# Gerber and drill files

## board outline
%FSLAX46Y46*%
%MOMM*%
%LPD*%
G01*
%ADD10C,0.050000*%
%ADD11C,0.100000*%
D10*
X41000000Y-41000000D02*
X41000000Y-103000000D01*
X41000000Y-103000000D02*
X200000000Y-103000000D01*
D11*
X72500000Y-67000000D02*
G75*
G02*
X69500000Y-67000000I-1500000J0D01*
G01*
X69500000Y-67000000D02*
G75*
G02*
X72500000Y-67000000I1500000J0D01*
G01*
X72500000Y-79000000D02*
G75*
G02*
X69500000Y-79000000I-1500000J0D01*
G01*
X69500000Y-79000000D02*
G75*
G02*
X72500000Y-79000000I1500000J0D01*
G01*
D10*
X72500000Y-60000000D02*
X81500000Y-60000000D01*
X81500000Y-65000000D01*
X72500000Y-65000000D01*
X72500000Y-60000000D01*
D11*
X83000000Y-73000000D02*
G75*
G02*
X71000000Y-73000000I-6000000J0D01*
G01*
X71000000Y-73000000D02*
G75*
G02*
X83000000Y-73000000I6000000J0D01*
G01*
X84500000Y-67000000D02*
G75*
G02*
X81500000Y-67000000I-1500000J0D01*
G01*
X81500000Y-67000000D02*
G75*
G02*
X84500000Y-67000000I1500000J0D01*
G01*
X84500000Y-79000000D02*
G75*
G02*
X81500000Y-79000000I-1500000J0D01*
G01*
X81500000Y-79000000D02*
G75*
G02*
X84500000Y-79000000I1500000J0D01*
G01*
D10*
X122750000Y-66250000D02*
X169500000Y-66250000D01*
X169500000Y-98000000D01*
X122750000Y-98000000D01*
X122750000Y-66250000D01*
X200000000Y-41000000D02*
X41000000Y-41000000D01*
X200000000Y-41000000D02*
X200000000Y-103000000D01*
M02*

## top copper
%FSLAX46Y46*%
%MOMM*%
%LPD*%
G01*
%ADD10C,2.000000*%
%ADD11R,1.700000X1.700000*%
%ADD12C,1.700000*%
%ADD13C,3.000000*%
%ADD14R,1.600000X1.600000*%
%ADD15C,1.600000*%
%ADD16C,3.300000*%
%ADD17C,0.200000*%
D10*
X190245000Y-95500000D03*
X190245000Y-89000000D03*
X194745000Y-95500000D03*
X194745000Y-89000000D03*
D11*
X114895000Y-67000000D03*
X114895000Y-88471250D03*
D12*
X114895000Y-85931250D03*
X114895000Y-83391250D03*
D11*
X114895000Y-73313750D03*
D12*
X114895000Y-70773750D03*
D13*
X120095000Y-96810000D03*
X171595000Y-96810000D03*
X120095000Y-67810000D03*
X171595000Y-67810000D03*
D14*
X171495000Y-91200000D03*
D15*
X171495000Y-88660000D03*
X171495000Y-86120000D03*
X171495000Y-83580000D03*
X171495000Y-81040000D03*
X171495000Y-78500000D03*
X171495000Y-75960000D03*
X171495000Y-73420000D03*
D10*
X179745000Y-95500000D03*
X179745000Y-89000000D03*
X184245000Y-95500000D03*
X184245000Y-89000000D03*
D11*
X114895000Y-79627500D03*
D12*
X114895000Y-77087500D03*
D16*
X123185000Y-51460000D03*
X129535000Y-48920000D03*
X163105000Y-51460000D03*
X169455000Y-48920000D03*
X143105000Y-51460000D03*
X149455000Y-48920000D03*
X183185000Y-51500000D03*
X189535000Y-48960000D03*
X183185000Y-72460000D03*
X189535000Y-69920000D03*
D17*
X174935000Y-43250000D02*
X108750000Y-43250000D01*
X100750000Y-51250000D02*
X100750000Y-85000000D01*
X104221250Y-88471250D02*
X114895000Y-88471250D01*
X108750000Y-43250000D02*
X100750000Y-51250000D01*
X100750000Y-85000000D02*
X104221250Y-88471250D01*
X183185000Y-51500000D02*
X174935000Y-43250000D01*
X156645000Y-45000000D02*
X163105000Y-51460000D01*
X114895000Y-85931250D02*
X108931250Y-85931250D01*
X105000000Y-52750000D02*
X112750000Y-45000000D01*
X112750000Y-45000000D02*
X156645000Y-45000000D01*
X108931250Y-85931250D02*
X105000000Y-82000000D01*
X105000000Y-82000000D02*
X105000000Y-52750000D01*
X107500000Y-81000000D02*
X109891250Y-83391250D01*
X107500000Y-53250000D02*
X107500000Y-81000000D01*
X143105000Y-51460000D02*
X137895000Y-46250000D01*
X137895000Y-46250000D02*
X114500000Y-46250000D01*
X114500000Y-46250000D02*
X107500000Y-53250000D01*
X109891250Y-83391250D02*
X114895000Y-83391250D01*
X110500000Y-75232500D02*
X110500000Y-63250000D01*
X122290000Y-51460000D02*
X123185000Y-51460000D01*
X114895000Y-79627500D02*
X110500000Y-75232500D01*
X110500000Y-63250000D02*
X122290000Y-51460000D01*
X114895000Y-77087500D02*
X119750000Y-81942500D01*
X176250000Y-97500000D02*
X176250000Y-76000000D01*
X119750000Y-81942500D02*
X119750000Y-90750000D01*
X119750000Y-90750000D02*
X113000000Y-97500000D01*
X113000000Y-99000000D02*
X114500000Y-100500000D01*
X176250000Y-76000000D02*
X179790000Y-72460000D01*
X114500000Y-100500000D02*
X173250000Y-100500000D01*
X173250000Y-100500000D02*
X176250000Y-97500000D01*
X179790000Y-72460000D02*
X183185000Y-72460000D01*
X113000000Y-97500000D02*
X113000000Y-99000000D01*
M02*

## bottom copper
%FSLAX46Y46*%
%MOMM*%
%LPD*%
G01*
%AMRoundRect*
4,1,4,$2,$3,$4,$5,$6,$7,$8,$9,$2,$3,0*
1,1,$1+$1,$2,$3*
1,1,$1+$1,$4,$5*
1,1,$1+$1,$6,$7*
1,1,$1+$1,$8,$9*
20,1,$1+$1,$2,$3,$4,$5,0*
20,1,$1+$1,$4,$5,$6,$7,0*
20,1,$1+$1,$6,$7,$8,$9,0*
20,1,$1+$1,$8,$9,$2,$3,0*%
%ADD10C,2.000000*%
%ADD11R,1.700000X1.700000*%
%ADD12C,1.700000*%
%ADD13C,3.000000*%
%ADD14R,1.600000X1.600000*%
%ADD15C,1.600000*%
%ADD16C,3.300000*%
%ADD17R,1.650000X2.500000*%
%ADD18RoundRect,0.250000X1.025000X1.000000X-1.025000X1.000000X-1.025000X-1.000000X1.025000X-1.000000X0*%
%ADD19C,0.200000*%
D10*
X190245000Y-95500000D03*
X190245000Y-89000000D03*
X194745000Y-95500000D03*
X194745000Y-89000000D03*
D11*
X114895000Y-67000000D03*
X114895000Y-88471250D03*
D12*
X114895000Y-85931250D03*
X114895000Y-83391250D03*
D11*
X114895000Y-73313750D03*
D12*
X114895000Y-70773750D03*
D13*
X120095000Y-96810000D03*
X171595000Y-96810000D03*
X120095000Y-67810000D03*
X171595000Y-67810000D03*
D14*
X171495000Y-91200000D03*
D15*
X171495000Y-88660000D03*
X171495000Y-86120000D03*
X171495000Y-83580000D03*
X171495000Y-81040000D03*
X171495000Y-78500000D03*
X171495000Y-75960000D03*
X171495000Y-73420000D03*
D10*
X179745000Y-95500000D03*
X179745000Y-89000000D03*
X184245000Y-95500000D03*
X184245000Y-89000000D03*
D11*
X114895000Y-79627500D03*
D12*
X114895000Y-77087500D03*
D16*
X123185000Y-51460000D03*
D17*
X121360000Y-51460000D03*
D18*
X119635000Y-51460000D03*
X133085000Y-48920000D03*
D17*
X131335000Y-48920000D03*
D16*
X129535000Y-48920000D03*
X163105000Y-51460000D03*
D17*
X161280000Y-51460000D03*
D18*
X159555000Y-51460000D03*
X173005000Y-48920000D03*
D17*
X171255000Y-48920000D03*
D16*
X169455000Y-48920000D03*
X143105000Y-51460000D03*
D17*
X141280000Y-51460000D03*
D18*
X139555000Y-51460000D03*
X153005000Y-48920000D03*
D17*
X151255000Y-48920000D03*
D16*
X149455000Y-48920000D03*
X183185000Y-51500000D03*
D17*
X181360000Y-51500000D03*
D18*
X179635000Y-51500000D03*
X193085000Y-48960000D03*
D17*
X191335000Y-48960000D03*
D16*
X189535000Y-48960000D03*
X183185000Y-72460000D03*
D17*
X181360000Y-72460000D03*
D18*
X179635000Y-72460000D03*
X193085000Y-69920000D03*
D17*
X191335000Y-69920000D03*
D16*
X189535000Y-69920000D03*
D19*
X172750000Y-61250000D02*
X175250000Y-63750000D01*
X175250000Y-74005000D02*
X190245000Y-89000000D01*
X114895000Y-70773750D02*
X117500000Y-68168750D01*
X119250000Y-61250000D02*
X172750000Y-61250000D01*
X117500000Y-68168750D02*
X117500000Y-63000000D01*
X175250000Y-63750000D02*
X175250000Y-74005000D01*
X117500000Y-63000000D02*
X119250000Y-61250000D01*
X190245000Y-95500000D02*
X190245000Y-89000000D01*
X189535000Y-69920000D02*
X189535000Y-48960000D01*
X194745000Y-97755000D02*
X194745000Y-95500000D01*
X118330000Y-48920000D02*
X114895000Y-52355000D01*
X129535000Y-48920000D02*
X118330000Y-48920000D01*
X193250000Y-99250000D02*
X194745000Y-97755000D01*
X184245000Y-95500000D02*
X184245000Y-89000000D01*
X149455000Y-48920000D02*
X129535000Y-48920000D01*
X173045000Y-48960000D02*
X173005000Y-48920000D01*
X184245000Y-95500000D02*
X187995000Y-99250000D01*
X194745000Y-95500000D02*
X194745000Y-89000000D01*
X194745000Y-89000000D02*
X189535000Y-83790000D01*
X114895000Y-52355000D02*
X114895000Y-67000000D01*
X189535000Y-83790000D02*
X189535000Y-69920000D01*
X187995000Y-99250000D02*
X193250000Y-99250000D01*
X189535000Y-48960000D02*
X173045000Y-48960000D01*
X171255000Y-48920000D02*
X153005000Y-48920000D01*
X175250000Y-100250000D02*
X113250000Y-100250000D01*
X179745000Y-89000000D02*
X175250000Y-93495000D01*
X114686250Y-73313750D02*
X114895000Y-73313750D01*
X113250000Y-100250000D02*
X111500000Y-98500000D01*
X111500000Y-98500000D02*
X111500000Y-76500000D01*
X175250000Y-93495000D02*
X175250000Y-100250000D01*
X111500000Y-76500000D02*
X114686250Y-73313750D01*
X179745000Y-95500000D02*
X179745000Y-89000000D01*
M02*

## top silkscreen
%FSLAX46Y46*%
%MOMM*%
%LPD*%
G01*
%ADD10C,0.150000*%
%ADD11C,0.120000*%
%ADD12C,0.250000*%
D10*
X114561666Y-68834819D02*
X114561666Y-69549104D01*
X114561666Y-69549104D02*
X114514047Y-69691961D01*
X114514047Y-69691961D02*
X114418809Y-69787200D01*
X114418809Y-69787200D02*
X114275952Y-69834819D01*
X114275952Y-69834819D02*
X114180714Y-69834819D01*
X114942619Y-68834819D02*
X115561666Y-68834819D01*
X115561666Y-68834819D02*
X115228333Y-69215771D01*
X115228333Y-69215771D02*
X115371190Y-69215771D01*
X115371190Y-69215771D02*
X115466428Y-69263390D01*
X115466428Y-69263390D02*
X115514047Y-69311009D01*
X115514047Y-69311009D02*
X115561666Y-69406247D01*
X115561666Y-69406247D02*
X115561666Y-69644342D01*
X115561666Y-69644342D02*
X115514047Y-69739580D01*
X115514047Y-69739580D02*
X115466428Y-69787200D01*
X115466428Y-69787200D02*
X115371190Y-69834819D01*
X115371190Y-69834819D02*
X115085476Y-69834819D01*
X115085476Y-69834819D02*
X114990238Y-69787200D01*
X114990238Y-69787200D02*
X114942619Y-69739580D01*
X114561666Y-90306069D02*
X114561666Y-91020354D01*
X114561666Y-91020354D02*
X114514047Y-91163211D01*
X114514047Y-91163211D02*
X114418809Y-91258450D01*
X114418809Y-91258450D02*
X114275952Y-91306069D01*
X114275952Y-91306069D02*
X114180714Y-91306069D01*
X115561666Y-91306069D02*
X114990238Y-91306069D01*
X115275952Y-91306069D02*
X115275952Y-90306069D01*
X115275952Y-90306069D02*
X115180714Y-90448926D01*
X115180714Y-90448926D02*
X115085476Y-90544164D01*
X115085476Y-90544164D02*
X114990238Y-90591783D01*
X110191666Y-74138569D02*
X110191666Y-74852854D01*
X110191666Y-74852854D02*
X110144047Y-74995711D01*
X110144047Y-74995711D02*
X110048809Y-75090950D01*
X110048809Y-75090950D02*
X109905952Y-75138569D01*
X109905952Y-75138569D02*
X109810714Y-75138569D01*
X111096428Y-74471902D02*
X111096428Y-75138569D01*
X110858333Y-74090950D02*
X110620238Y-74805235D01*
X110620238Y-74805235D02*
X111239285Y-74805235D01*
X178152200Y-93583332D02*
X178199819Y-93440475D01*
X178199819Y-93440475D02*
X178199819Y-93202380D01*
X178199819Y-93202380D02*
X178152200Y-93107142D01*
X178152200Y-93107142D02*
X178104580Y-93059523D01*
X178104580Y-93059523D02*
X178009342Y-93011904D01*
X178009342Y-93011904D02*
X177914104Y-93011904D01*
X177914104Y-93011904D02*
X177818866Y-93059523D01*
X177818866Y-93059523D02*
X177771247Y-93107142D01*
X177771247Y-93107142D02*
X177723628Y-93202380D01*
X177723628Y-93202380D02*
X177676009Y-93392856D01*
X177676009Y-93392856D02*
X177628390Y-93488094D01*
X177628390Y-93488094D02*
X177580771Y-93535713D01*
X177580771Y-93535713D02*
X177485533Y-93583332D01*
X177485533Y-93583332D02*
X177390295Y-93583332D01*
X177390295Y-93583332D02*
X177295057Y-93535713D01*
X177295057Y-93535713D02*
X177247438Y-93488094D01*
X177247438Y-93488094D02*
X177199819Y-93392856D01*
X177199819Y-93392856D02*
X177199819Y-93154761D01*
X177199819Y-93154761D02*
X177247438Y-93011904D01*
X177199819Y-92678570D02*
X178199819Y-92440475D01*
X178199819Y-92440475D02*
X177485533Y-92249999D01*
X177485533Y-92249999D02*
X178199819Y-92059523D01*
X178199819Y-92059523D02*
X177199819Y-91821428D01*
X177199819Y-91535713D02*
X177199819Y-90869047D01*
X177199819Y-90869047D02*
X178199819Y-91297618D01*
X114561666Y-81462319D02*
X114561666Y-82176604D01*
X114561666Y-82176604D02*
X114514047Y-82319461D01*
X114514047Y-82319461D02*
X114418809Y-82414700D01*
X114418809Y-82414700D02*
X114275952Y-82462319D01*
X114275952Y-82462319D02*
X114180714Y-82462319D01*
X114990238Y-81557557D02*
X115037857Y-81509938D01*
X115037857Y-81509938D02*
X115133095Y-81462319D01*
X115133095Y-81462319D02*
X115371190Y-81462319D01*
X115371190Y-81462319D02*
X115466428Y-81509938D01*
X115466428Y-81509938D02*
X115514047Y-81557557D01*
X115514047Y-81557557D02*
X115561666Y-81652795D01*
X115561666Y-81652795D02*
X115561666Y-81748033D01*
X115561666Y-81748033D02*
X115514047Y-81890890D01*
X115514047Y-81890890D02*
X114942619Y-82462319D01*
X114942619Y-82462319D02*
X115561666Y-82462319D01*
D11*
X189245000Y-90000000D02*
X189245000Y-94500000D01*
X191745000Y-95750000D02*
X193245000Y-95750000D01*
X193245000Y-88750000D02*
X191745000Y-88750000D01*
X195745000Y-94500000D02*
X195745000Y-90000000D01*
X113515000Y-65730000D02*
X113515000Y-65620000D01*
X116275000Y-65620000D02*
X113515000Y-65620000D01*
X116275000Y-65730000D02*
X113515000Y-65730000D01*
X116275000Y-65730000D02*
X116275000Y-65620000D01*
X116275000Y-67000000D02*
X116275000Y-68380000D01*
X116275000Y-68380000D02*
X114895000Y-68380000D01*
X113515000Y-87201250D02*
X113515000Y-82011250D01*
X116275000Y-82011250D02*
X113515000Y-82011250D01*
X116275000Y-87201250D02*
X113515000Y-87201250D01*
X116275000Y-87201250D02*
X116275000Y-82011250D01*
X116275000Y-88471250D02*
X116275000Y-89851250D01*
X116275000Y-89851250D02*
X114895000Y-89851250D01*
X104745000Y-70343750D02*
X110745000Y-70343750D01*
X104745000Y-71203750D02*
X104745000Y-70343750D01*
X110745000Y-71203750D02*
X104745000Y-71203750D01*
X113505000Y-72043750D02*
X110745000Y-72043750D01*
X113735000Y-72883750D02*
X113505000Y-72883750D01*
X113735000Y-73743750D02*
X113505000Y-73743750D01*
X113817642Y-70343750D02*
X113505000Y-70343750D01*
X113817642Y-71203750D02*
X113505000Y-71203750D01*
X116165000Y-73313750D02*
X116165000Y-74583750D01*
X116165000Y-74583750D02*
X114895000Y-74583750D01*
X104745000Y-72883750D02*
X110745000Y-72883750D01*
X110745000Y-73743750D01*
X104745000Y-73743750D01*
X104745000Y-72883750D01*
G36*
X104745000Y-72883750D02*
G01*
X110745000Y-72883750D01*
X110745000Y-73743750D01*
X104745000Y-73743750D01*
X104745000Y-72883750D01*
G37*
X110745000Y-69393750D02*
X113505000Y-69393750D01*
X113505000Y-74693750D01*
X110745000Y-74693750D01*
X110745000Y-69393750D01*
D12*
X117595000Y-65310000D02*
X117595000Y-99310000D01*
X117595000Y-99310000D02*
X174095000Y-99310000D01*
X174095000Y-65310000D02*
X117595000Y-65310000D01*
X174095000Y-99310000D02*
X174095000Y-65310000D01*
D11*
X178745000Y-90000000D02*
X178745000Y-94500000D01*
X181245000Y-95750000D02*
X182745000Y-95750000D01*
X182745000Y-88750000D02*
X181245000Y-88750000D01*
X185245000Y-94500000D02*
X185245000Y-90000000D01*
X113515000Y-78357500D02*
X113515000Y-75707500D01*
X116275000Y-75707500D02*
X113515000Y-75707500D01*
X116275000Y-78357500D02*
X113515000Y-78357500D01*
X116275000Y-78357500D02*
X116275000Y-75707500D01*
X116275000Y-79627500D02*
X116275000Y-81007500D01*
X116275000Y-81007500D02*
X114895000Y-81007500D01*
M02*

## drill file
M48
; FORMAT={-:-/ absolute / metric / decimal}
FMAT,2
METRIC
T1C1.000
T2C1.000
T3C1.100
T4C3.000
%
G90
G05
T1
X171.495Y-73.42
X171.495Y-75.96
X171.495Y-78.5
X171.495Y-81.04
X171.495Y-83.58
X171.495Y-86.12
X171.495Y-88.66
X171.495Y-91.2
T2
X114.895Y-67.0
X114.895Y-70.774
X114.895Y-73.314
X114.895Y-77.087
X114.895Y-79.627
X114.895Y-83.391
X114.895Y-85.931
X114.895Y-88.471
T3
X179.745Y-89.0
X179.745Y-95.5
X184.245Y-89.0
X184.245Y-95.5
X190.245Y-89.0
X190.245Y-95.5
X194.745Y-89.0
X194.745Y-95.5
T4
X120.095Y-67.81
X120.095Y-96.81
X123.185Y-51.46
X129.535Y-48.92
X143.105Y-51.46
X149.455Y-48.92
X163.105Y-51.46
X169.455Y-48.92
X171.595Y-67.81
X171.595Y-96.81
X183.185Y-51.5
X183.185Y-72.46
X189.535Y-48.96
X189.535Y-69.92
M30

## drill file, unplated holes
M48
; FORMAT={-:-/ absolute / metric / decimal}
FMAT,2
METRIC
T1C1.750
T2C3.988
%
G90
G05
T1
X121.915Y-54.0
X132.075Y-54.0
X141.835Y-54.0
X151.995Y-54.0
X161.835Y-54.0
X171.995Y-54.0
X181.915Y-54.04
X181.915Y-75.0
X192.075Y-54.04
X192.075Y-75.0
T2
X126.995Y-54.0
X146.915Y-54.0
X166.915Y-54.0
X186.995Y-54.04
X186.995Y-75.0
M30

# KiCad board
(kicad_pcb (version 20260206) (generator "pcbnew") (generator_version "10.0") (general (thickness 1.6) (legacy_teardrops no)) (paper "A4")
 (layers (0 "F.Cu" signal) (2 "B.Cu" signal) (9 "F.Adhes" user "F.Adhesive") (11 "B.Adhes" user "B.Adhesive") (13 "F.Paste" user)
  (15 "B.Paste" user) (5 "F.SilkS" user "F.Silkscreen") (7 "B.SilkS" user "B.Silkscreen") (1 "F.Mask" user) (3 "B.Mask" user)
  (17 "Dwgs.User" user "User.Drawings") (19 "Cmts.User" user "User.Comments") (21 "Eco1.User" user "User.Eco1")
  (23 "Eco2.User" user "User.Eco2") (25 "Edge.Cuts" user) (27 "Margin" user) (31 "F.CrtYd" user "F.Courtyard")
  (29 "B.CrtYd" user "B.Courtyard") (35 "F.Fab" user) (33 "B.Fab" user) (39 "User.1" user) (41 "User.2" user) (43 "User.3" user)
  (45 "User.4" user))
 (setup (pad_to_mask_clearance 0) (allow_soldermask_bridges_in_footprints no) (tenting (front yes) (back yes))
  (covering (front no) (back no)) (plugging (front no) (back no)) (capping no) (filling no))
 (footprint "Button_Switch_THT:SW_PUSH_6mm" (layer "F.Cu") (at 190.245 95.5 90)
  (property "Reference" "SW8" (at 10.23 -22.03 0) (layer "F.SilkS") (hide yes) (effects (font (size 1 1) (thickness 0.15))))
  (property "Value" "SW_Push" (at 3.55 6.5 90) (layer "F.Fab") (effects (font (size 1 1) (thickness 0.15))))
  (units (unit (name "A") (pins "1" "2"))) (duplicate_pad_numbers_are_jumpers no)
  (fp_line (start 5.5 -1) (end 1 -1) (stroke (width 0.12) (type solid)) (layer "F.SilkS"))
  (fp_line (start -0.25 1.5) (end -0.25 3) (stroke (width 0.12) (type solid)) (layer "F.SilkS"))
  (fp_line (start 6.75 3) (end 6.75 1.5) (stroke (width 0.12) (type solid)) (layer "F.SilkS"))
  (fp_line (start 1 5.5) (end 5.5 5.5) (stroke (width 0.12) (type solid)) (layer "F.SilkS"))
  (pad "1" thru_hole circle (at 0 0 180) (size 2 2) (drill 1.1) (layers "*.Cu" "*.Mask") (remove_unused_layers no) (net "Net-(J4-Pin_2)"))
  (pad "1" thru_hole circle (at 6.5 0 180) (size 2 2) (drill 1.1) (layers "*.Cu" "*.Mask") (remove_unused_layers no) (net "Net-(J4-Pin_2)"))
  (pad "2" thru_hole circle (at 0 4.5 180) (size 2 2) (drill 1.1) (layers "*.Cu" "*.Mask") (remove_unused_layers no) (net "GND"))
  (pad "2" thru_hole circle (at 6.5 4.5 180) (size 2 2) (drill 1.1) (layers "*.Cu" "*.Mask") (remove_unused_layers no) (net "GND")))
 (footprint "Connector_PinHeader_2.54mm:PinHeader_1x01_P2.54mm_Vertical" (layer "F.Cu") (at 114.895 67 180)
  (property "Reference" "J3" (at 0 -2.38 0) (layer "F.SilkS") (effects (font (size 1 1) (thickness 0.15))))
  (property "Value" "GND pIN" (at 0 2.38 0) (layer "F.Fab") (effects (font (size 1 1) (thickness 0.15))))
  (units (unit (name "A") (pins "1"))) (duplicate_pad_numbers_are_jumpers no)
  (fp_line (start 1.38 1.27) (end 1.38 1.38) (stroke (width 0.12) (type solid)) (layer "F.SilkS"))
  (fp_line (start -1.38 1.38) (end 1.38 1.38) (stroke (width 0.12) (type solid)) (layer "F.SilkS"))
  (fp_line (start -1.38 1.27) (end 1.38 1.27) (stroke (width 0.12) (type solid)) (layer "F.SilkS"))
  (fp_line (start -1.38 1.27) (end -1.38 1.38) (stroke (width 0.12) (type solid)) (layer "F.SilkS"))
  (fp_line (start -1.38 0) (end -1.38 -1.38) (stroke (width 0.12) (type solid)) (layer "F.SilkS"))
  (fp_line (start -1.38 -1.38) (end 0 -1.38) (stroke (width 0.12) (type solid)) (layer "F.SilkS"))
  (pad "1" thru_hole rect (at 0 0 180) (size 1.7 1.7) (drill 1) (layers "*.Cu" "*.Mask") (remove_unused_layers no) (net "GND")))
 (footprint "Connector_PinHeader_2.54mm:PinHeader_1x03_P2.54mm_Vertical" (layer "F.Cu") (at 114.895 88.47125 180)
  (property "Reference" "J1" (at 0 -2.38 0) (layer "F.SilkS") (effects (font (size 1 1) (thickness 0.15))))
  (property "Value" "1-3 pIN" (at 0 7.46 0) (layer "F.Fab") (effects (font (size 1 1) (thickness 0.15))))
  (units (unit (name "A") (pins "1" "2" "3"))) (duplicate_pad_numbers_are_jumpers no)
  (fp_line (start 1.38 1.27) (end 1.38 6.46) (stroke (width 0.12) (type solid)) (layer "F.SilkS"))
  (fp_line (start -1.38 6.46) (end 1.38 6.46) (stroke (width 0.12) (type solid)) (layer "F.SilkS"))
  (fp_line (start -1.38 1.27) (end 1.38 1.27) (stroke (width 0.12) (type solid)) (layer "F.SilkS"))
  (fp_line (start -1.38 1.27) (end -1.38 6.46) (stroke (width 0.12) (type solid)) (layer "F.SilkS"))
  (fp_line (start -1.38 0) (end -1.38 -1.38) (stroke (width 0.12) (type solid)) (layer "F.SilkS"))
  (fp_line (start -1.38 -1.38) (end 0 -1.38) (stroke (width 0.12) (type solid)) (layer "F.SilkS"))
  (pad "1" thru_hole rect (at 0 0 180) (size 1.7 1.7) (drill 1) (layers "*.Cu" "*.Mask") (remove_unused_layers no) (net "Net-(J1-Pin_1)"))
  (pad "2" thru_hole circle (at 0 2.54 180) (size 1.7 1.7) (drill 1) (layers "*.Cu" "*.Mask") (remove_unused_layers no)
   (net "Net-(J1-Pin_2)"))
  (pad "3" thru_hole circle (at 0 5.08 180) (size 1.7 1.7) (drill 1) (layers "*.Cu" "*.Mask") (remove_unused_layers no)
   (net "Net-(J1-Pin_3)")))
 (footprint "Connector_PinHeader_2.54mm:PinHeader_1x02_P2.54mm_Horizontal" (layer "F.Cu") (at 114.895 73.31375 180)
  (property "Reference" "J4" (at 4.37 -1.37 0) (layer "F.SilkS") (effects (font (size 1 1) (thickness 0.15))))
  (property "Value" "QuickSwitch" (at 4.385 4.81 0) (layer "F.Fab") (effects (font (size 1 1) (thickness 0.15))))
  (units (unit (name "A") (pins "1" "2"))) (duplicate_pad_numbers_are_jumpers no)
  (fp_line (start 10.15 2.97) (end 4.15 2.97) (stroke (width 0.12) (type solid)) (layer "F.SilkS"))
  (fp_line (start 10.15 2.11) (end 10.15 2.97) (stroke (width 0.12) (type solid)) (layer "F.SilkS"))
  (fp_line (start 4.15 2.11) (end 10.15 2.11) (stroke (width 0.12) (type solid)) (layer "F.SilkS"))
  (fp_line (start 1.39 1.27) (end 4.15 1.27) (stroke (width 0.12) (type solid)) (layer "F.SilkS"))
  (fp_line (start 1.16 0.43) (end 1.39 0.43) (stroke (width 0.12) (type solid)) (layer "F.SilkS"))
  (fp_line (start 1.16 -0.43) (end 1.39 -0.43) (stroke (width 0.12) (type solid)) (layer "F.SilkS"))
  (fp_line (start 1.077358 2.97) (end 1.39 2.97) (stroke (width 0.12) (type solid)) (layer "F.SilkS"))
  (fp_line (start 1.077358 2.11) (end 1.39 2.11) (stroke (width 0.12) (type solid)) (layer "F.SilkS"))
  (fp_line (start -1.27 0) (end -1.27 -1.27) (stroke (width 0.12) (type solid)) (layer "F.SilkS"))
  (fp_line (start -1.27 -1.27) (end 0 -1.27) (stroke (width 0.12) (type solid)) (layer "F.SilkS"))
  (fp_rect (start 4.15 -0.43) (end 10.15 0.43) (stroke (width 0.12) (type solid)) (fill yes) (layer "F.SilkS"))
  (fp_rect (start 1.39 -1.38) (end 4.15 3.92) (stroke (width 0.12) (type solid)) (fill no) (layer "F.SilkS"))
  (pad "1" thru_hole rect (at 0 0 180) (size 1.7 1.7) (drill 1) (layers "*.Cu" "*.Mask") (remove_unused_layers no) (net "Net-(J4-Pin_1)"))
  (pad "2" thru_hole circle (at 0 2.54 180) (size 1.7 1.7) (drill 1) (layers "*.Cu" "*.Mask") (remove_unused_layers no)
   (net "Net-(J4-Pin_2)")))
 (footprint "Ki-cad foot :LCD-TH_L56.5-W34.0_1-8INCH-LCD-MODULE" (layer "F.Cu") (at 171.495 82.31 90)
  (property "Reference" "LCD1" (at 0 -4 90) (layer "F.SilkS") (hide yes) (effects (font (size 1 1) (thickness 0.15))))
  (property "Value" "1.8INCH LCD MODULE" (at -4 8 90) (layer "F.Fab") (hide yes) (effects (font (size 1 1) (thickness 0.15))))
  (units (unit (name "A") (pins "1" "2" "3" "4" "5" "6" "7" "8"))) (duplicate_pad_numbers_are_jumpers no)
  (fp_line (start 17 -53.9) (end -17 -53.9) (stroke (width 0.25) (type solid)) (layer "F.SilkS"))
  (fp_line (start -17 -53.9) (end -17 2.6) (stroke (width 0.25) (type solid)) (layer "F.SilkS"))
  (fp_line (start 17 2.6) (end 17 -53.9) (stroke (width 0.25) (type solid)) (layer "F.SilkS"))
  (fp_line (start -17 2.6) (end 17 2.6) (stroke (width 0.25) (type solid)) (layer "F.SilkS"))
  (pad "" thru_hole circle (at -14.5 -51.4 90) (size 3 3) (drill 3) (layers "*.Cu" "*.Mask") (remove_unused_layers no))
  (pad "" thru_hole circle (at -14.5 0.1 90) (size 3 3) (drill 3) (layers "*.Cu" "*.Mask") (remove_unused_layers no))
  (pad "" thru_hole circle (at 14.5 -51.4 90) (size 3 3) (drill 3) (layers "*.Cu" "*.Mask") (remove_unused_layers no))
  (pad "" thru_hole circle (at 14.5 0.1 90) (size 3 3) (drill 3) (layers "*.Cu" "*.Mask") (remove_unused_layers no))
  (pad "1" thru_hole rect (at -8.89 0 90) (size 1.6 1.6) (drill 0.999998) (layers "*.Cu" "*.Mask") (remove_unused_layers no)
   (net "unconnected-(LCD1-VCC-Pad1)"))
  (pad "2" thru_hole circle (at -6.35 0 90) (size 1.6 1.6) (drill 0.999998) (layers "*.Cu" "*.Mask") (remove_unused_layers no)
   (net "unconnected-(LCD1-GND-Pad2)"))
  (pad "3" thru_hole circle (at -3.81 0 90) (size 1.6 1.6) (drill 0.999998) (layers "*.Cu" "*.Mask") (remove_unused_layers no)
   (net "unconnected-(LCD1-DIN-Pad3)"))
  (pad "4" thru_hole circle (at -1.27 0 90) (size 1.6 1.6) (drill 0.999998) (layers "*.Cu" "*.Mask") (remove_unused_layers no)
   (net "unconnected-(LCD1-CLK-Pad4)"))
  (pad "5" thru_hole circle (at 1.27 0 90) (size 1.6 1.6) (drill 0.999998) (layers "*.Cu" "*.Mask") (remove_unused_layers no)
   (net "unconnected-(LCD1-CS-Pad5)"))
  (pad "6" thru_hole circle (at 3.81 0 90) (size 1.6 1.6) (drill 0.999998) (layers "*.Cu" "*.Mask") (remove_unused_layers no)
   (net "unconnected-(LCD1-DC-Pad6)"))
  (pad "7" thru_hole circle (at 6.35 0 90) (size 1.6 1.6) (drill 0.999998) (layers "*.Cu" "*.Mask") (remove_unused_layers no)
   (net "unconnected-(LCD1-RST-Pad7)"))
  (pad "8" thru_hole circle (at 8.89 0 90) (size 1.6 1.6) (drill 0.999998) (layers "*.Cu" "*.Mask") (remove_unused_layers no)
   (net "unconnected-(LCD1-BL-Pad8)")))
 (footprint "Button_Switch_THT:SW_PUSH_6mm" (layer "F.Cu") (at 179.745 95.5 90)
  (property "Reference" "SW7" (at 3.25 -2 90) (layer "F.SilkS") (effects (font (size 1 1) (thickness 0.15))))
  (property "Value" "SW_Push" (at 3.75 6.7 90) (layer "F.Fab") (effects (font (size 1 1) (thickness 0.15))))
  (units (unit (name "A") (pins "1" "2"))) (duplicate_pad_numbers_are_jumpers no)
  (fp_line (start 5.5 -1) (end 1 -1) (stroke (width 0.12) (type solid)) (layer "F.SilkS"))
  (fp_line (start -0.25 1.5) (end -0.25 3) (stroke (width 0.12) (type solid)) (layer "F.SilkS"))
  (fp_line (start 6.75 3) (end 6.75 1.5) (stroke (width 0.12) (type solid)) (layer "F.SilkS"))
  (fp_line (start 1 5.5) (end 5.5 5.5) (stroke (width 0.12) (type solid)) (layer "F.SilkS"))
  (pad "1" thru_hole circle (at 0 0 180) (size 2 2) (drill 1.1) (layers "*.Cu" "*.Mask") (remove_unused_layers no) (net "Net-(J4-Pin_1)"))
  (pad "1" thru_hole circle (at 6.5 0 180) (size 2 2) (drill 1.1) (layers "*.Cu" "*.Mask") (remove_unused_layers no) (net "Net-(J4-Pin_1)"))
  (pad "2" thru_hole circle (at 0 4.5 180) (size 2 2) (drill 1.1) (layers "*.Cu" "*.Mask") (remove_unused_layers no) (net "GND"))
  (pad "2" thru_hole circle (at 6.5 4.5 180) (size 2 2) (drill 1.1) (layers "*.Cu" "*.Mask") (remove_unused_layers no) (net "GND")))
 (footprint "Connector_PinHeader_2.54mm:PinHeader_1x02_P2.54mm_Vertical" (layer "F.Cu") (at 114.895 79.6275 180)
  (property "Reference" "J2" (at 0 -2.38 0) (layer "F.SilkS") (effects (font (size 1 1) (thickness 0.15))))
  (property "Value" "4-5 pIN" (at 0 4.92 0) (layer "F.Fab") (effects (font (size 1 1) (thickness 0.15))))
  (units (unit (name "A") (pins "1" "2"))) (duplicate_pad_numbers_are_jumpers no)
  (fp_line (start 1.38 1.27) (end 1.38 3.92) (stroke (width 0.12) (type solid)) (layer "F.SilkS"))
  (fp_line (start -1.38 3.92) (end 1.38 3.92) (stroke (width 0.12) (type solid)) (layer "F.SilkS"))
  (fp_line (start -1.38 1.27) (end 1.38 1.27) (stroke (width 0.12) (type solid)) (layer "F.SilkS"))
  (fp_line (start -1.38 1.27) (end -1.38 3.92) (stroke (width 0.12) (type solid)) (layer "F.SilkS"))
  (fp_line (start -1.38 0) (end -1.38 -1.38) (stroke (width 0.12) (type solid)) (layer "F.SilkS"))
  (fp_line (start -1.38 -1.38) (end 0 -1.38) (stroke (width 0.12) (type solid)) (layer "F.SilkS"))
  (pad "1" thru_hole rect (at 0 0 180) (size 1.7 1.7) (drill 1) (layers "*.Cu" "*.Mask") (remove_unused_layers no) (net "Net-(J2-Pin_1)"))
  (pad "2" thru_hole circle (at 0 2.54 180) (size 1.7 1.7) (drill 1) (layers "*.Cu" "*.Mask") (remove_unused_layers no)
   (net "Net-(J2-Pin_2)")))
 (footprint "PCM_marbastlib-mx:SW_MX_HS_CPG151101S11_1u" (layer "B.Cu") (at 126.995 54 180)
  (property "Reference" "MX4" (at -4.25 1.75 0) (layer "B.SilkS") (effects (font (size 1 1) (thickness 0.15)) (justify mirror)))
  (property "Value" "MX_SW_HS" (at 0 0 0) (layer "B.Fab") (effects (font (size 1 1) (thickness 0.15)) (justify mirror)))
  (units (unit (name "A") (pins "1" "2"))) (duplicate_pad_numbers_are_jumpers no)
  (pad "" np_thru_hole circle (at -5.08 0 180) (size 1.75 1.75) (drill 1.75) (layers "*.Cu" "*.Mask"))
  (pad "" np_thru_hole circle (at 0 0 180) (size 3.9878 3.9878) (drill 3.9878) (layers "*.Cu" "*.Mask"))
  (pad "" np_thru_hole circle (at 5.08 0 180) (size 1.75 1.75) (drill 1.75) (layers "*.Cu" "*.Mask"))
  (pad "1" thru_hole circle (at 3.81 2.54 180) (size 3.3 3.3) (drill 3) (layers "*.Cu" "*.Mask") (remove_unused_layers no)
   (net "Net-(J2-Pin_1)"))
  (pad "1" smd rect (at 5.635 2.54) (size 1.65 2.5) (layers "B.Cu") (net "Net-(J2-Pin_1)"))
  (pad "1" smd roundrect (at 7.36 2.54 180) (size 2.55 2.5) (layers "B.Cu" "B.Mask" "B.Paste") (roundrect_rratio 0.1) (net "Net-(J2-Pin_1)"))
  (pad "2" smd roundrect (at -6.09 5.08 180) (size 2.55 2.5) (layers "B.Cu" "B.Mask" "B.Paste") (roundrect_rratio 0.1) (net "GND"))
  (pad "2" smd rect (at -4.34 5.08 180) (size 1.65 2.5) (layers "B.Cu") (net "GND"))
  (pad "2" thru_hole circle (at -2.54 5.08 180) (size 3.3 3.3) (drill 3) (layers "*.Cu" "*.Mask") (remove_unused_layers no) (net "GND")))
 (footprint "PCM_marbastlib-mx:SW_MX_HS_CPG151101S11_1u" (layer "B.Cu") (at 166.915 54 180)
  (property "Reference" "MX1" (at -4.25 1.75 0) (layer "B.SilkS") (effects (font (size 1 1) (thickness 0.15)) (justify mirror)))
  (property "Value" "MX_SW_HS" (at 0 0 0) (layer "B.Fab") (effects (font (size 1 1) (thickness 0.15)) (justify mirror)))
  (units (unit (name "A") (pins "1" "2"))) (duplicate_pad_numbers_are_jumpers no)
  (pad "" np_thru_hole circle (at -5.08 0 180) (size 1.75 1.75) (drill 1.75) (layers "*.Cu" "*.Mask"))
  (pad "" np_thru_hole circle (at 0 0 180) (size 3.9878 3.9878) (drill 3.9878) (layers "*.Cu" "*.Mask"))
  (pad "" np_thru_hole circle (at 5.08 0 180) (size 1.75 1.75) (drill 1.75) (layers "*.Cu" "*.Mask"))
  (pad "1" thru_hole circle (at 3.81 2.54 180) (size 3.3 3.3) (drill 3) (layers "*.Cu" "*.Mask") (remove_unused_layers no)
   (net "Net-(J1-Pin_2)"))
  (pad "1" smd rect (at 5.635 2.54) (size 1.65 2.5) (layers "B.Cu") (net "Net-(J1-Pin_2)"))
  (pad "1" smd roundrect (at 7.36 2.54 180) (size 2.55 2.5) (layers "B.Cu" "B.Mask" "B.Paste") (roundrect_rratio 0.1) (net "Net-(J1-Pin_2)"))
  (pad "2" smd roundrect (at -6.09 5.08 180) (size 2.55 2.5) (layers "B.Cu" "B.Mask" "B.Paste") (roundrect_rratio 0.1) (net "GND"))
  (pad "2" smd rect (at -4.34 5.08 180) (size 1.65 2.5) (layers "B.Cu") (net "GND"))
  (pad "2" thru_hole circle (at -2.54 5.08 180) (size 3.3 3.3) (drill 3) (layers "*.Cu" "*.Mask") (remove_unused_layers no) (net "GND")))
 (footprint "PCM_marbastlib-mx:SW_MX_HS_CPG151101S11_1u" (layer "B.Cu") (at 146.915 54 180)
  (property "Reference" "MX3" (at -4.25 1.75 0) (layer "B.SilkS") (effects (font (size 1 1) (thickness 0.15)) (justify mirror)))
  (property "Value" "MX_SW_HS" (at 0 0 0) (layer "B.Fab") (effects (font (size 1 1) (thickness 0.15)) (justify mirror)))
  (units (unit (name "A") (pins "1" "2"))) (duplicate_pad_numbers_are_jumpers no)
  (pad "" np_thru_hole circle (at -5.08 0 180) (size 1.75 1.75) (drill 1.75) (layers "*.Cu" "*.Mask"))
  (pad "" np_thru_hole circle (at 0 0 180) (size 3.9878 3.9878) (drill 3.9878) (layers "*.Cu" "*.Mask"))
  (pad "" np_thru_hole circle (at 5.08 0 180) (size 1.75 1.75) (drill 1.75) (layers "*.Cu" "*.Mask"))
  (pad "1" thru_hole circle (at 3.81 2.54 180) (size 3.3 3.3) (drill 3) (layers "*.Cu" "*.Mask") (remove_unused_layers no)
   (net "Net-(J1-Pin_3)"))
  (pad "1" smd rect (at 5.635 2.54) (size 1.65 2.5) (layers "B.Cu") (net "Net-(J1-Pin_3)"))
  (pad "1" smd roundrect (at 7.36 2.54 180) (size 2.55 2.5) (layers "B.Cu" "B.Mask" "B.Paste") (roundrect_rratio 0.1) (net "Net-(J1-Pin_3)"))
  (pad "2" smd roundrect (at -6.09 5.08 180) (size 2.55 2.5) (layers "B.Cu" "B.Mask" "B.Paste") (roundrect_rratio 0.1) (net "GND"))
  (pad "2" smd rect (at -4.34 5.08 180) (size 1.65 2.5) (layers "B.Cu") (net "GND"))
  (pad "2" thru_hole circle (at -2.54 5.08 180) (size 3.3 3.3) (drill 3) (layers "*.Cu" "*.Mask") (remove_unused_layers no) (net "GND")))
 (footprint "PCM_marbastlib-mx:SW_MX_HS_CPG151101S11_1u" (layer "B.Cu") (at 186.995 54.04 180)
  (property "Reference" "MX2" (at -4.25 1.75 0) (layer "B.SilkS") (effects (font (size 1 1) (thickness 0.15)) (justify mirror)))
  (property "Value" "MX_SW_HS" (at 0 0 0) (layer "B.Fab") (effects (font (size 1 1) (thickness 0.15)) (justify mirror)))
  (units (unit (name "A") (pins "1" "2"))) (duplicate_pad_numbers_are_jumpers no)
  (pad "" np_thru_hole circle (at -5.08 0 180) (size 1.75 1.75) (drill 1.75) (layers "*.Cu" "*.Mask"))
  (pad "" np_thru_hole circle (at 0 0 180) (size 3.9878 3.9878) (drill 3.9878) (layers "*.Cu" "*.Mask"))
  (pad "" np_thru_hole circle (at 5.08 0 180) (size 1.75 1.75) (drill 1.75) (layers "*.Cu" "*.Mask"))
  (pad "1" thru_hole circle (at 3.81 2.54 180) (size 3.3 3.3) (drill 3) (layers "*.Cu" "*.Mask") (remove_unused_layers no)
   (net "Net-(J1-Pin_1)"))
  (pad "1" smd rect (at 5.635 2.54) (size 1.65 2.5) (layers "B.Cu") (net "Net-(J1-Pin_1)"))
  (pad "1" smd roundrect (at 7.36 2.54 180) (size 2.55 2.5) (layers "B.Cu" "B.Mask" "B.Paste") (roundrect_rratio 0.1) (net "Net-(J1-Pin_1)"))
  (pad "2" smd roundrect (at -6.09 5.08 180) (size 2.55 2.5) (layers "B.Cu" "B.Mask" "B.Paste") (roundrect_rratio 0.1) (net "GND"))
  (pad "2" smd rect (at -4.34 5.08 180) (size 1.65 2.5) (layers "B.Cu") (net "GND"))
  (pad "2" thru_hole circle (at -2.54 5.08 180) (size 3.3 3.3) (drill 3) (layers "*.Cu" "*.Mask") (remove_unused_layers no) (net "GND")))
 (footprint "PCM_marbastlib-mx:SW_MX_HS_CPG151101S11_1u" (layer "B.Cu") (at 186.995 75 180)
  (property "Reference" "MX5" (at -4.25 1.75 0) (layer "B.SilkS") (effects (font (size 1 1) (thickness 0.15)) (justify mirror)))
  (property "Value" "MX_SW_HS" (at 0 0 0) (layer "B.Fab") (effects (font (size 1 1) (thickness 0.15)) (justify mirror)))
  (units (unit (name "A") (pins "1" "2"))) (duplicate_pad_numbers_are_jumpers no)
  (pad "" np_thru_hole circle (at -5.08 0 180) (size 1.75 1.75) (drill 1.75) (layers "*.Cu" "*.Mask"))
  (pad "" np_thru_hole circle (at 0 0 180) (size 3.9878 3.9878) (drill 3.9878) (layers "*.Cu" "*.Mask"))
  (pad "" np_thru_hole circle (at 5.08 0 180) (size 1.75 1.75) (drill 1.75) (layers "*.Cu" "*.Mask"))
  (pad "1" thru_hole circle (at 3.81 2.54 180) (size 3.3 3.3) (drill 3) (layers "*.Cu" "*.Mask") (remove_unused_layers no)
   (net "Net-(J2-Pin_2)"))
  (pad "1" smd rect (at 5.635 2.54) (size 1.65 2.5) (layers "B.Cu") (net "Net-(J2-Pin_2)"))
  (pad "1" smd roundrect (at 7.36 2.54 180) (size 2.55 2.5) (layers "B.Cu" "B.Mask" "B.Paste") (roundrect_rratio 0.1) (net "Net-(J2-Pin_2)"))
  (pad "2" smd roundrect (at -6.09 5.08 180) (size 2.55 2.5) (layers "B.Cu" "B.Mask" "B.Paste") (roundrect_rratio 0.1) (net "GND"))
  (pad "2" smd rect (at -4.34 5.08 180) (size 1.65 2.5) (layers "B.Cu") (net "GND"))
  (pad "2" thru_hole circle (at -2.54 5.08 180) (size 3.3 3.3) (drill 3) (layers "*.Cu" "*.Mask") (remove_unused_layers no) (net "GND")))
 (gr_line (start 41 41) (end 41 103) (stroke (width 0.05) (type default)) (layer "Edge.Cuts"))
 (gr_line (start 41 103) (end 200 103) (stroke (width 0.05) (type default)) (layer "Edge.Cuts"))
 (gr_circle (center 71 67) (end 72.5 67) (stroke (width 0.1) (type solid)) (fill no) (layer "Edge.Cuts"))
 (gr_circle (center 71 79) (end 72.5 79) (stroke (width 0.1) (type solid)) (fill no) (layer "Edge.Cuts"))
 (gr_rect (start 72.5 60) (end 81.5 65) (stroke (width 0.05) (type solid)) (fill no) (layer "Edge.Cuts"))
 (gr_circle (center 77 73) (end 83 73) (stroke (width 0.1) (type solid)) (fill no) (layer "Edge.Cuts"))
 (gr_circle (center 83 67) (end 84.5 67) (stroke (width 0.1) (type solid)) (fill no) (layer "Edge.Cuts"))
 (gr_circle (center 83 79) (end 84.5 79) (stroke (width 0.1) (type solid)) (fill no) (layer "Edge.Cuts"))
 (gr_rect (start 122.75 66.25) (end 169.5 98) (stroke (width 0.05) (type default)) (fill no) (layer "Edge.Cuts"))
 (gr_line (start 200 41) (end 41 41) (stroke (width 0.05) (type default)) (layer "Edge.Cuts"))
 (gr_line (start 200 41) (end 200 103) (stroke (width 0.05) (type default)) (layer "Edge.Cuts"))
 (segment (start 172.75 61.25) (end 175.25 63.75) (width 0.2) (layer "B.Cu") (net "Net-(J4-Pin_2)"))
 (segment (start 175.25 74.005) (end 190.245 89) (width 0.2) (layer "B.Cu") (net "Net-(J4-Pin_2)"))
 (segment (start 114.895 70.77375) (end 117.5 68.16875) (width 0.2) (layer "B.Cu") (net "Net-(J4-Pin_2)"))
 (segment (start 119.25 61.25) (end 172.75 61.25) (width 0.2) (layer "B.Cu") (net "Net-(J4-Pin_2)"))
 (segment (start 117.5 68.16875) (end 117.5 63) (width 0.2) (layer "B.Cu") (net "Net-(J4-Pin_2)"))
 (segment (start 175.25 63.75) (end 175.25 74.005) (width 0.2) (layer "B.Cu") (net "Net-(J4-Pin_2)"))
 (segment (start 117.5 63) (end 119.25 61.25) (width 0.2) (layer "B.Cu") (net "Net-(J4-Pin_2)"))
 (segment (start 190.245 95.5) (end 190.245 89) (width 0.2) (layer "B.Cu") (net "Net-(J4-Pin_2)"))
 (segment (start 189.535 69.92) (end 189.535 48.96) (width 0.2) (layer "B.Cu") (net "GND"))
 (segment (start 194.745 97.755) (end 194.745 95.5) (width 0.2) (layer "B.Cu") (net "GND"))
 (segment (start 118.33 48.92) (end 114.895 52.355) (width 0.2) (layer "B.Cu") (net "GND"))
 (segment (start 129.535 48.92) (end 118.33 48.92) (width 0.2) (layer "B.Cu") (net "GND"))
 (segment (start 193.25 99.25) (end 194.745 97.755) (width 0.2) (layer "B.Cu") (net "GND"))
 (segment (start 184.245 95.5) (end 184.245 89) (width 0.2) (layer "B.Cu") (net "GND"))
 (segment (start 149.455 48.92) (end 129.535 48.92) (width 0.2) (layer "B.Cu") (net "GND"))
 (segment (start 173.045 48.96) (end 173.005 48.92) (width 0.2) (layer "B.Cu") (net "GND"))
 (segment (start 184.245 95.5) (end 187.995 99.25) (width 0.2) (layer "B.Cu") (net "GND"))
 (segment (start 194.745 95.5) (end 194.745 89) (width 0.2) (layer "B.Cu") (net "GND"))
 (segment (start 194.745 89) (end 189.535 83.79) (width 0.2) (layer "B.Cu") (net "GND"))
 (segment (start 114.895 52.355) (end 114.895 67) (width 0.2) (layer "B.Cu") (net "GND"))
 (segment (start 189.535 83.79) (end 189.535 69.92) (width 0.2) (layer "B.Cu") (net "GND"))
 (segment (start 187.995 99.25) (end 193.25 99.25) (width 0.2) (layer "B.Cu") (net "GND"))
 (segment (start 189.535 48.96) (end 173.045 48.96) (width 0.2) (layer "B.Cu") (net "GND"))
 (segment (start 171.255 48.92) (end 153.005 48.92) (width 0.2) (layer "B.Cu") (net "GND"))
 (segment (start 174.935 43.25) (end 108.75 43.25) (width 0.2) (layer "F.Cu") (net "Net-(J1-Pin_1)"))
 (segment (start 100.75 51.25) (end 100.75 85) (width 0.2) (layer "F.Cu") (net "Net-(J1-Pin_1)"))
 (segment (start 104.22125 88.47125) (end 114.895 88.47125) (width 0.2) (layer "F.Cu") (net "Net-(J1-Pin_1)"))
 (segment (start 108.75 43.25) (end 100.75 51.25) (width 0.2) (layer "F.Cu") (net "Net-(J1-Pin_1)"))
 (segment (start 100.75 85) (end 104.22125 88.47125) (width 0.2) (layer "F.Cu") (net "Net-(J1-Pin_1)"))
 (segment (start 183.185 51.5) (end 174.935 43.25) (width 0.2) (layer "F.Cu") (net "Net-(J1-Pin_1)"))
 (segment (start 156.645 45) (end 163.105 51.46) (width 0.2) (layer "F.Cu") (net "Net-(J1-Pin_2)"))
 (segment (start 114.895 85.93125) (end 108.93125 85.93125) (width 0.2) (layer "F.Cu") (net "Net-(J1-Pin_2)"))
 (segment (start 105 52.75) (end 112.75 45) (width 0.2) (layer "F.Cu") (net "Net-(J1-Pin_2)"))
 (segment (start 112.75 45) (end 156.645 45) (width 0.2) (layer "F.Cu") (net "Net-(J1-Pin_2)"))
 (segment (start 108.93125 85.93125) (end 105 82) (width 0.2) (layer "F.Cu") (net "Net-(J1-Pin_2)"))
 (segment (start 105 82) (end 105 52.75) (width 0.2) (layer "F.Cu") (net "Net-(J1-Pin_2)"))
 (segment (start 107.5 81) (end 109.89125 83.39125) (width 0.2) (layer "F.Cu") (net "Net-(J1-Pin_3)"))
 (segment (start 107.5 53.25) (end 107.5 81) (width 0.2) (layer "F.Cu") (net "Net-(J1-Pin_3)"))
 (segment (start 143.105 51.46) (end 137.895 46.25) (width 0.2) (layer "F.Cu") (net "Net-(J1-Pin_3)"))
 (segment (start 137.895 46.25) (end 114.5 46.25) (width 0.2) (layer "F.Cu") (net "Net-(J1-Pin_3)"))
 (segment (start 114.5 46.25) (end 107.5 53.25) (width 0.2) (layer "F.Cu") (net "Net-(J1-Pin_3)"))
 (segment (start 109.89125 83.39125) (end 114.895 83.39125) (width 0.2) (layer "F.Cu") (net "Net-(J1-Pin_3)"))
 (segment (start 175.25 100.25) (end 113.25 100.25) (width 0.2) (layer "B.Cu") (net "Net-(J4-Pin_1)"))
 (segment (start 179.745 89) (end 175.25 93.495) (width 0.2) (layer "B.Cu") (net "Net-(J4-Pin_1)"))
 (segment (start 114.68625 73.31375) (end 114.895 73.31375) (width 0.2) (layer "B.Cu") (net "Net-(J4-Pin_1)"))
 (segment (start 113.25 100.25) (end 111.5 98.5) (width 0.2) (layer "B.Cu") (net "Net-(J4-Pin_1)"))
 (segment (start 111.5 98.5) (end 111.5 76.5) (width 0.2) (layer "B.Cu") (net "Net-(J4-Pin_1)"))
 (segment (start 175.25 93.495) (end 175.25 100.25) (width 0.2) (layer "B.Cu") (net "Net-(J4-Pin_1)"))
 (segment (start 111.5 76.5) (end 114.68625 73.31375) (width 0.2) (layer "B.Cu") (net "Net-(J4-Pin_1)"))
 (segment (start 179.745 95.5) (end 179.745 89) (width 0.2) (layer "B.Cu") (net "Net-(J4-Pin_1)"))
 (segment (start 110.5 75.2325) (end 110.5 63.25) (width 0.2) (layer "F.Cu") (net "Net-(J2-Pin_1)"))
 (segment (start 122.29 51.46) (end 123.185 51.46) (width 0.2) (layer "F.Cu") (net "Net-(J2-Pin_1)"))
 (segment (start 114.895 79.6275) (end 110.5 75.2325) (width 0.2) (layer "F.Cu") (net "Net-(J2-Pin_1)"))
 (segment (start 110.5 63.25) (end 122.29 51.46) (width 0.2) (layer "F.Cu") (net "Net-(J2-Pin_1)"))
 (segment (start 114.895 77.0875) (end 119.75 81.9425) (width 0.2) (layer "F.Cu") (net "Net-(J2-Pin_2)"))
 (segment (start 176.25 97.5) (end 176.25 76) (width 0.2) (layer "F.Cu") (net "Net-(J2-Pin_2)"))
 (segment (start 119.75 81.9425) (end 119.75 90.75) (width 0.2) (layer "F.Cu") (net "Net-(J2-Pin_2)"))
 (segment (start 119.75 90.75) (end 113 97.5) (width 0.2) (layer "F.Cu") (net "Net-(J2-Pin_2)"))
 (segment (start 113 99) (end 114.5 100.5) (width 0.2) (layer "F.Cu") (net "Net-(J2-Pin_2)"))
 (segment (start 176.25 76) (end 179.79 72.46) (width 0.2) (layer "F.Cu") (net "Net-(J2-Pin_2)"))
 (segment (start 114.5 100.5) (end 173.25 100.5) (width 0.2) (layer "F.Cu") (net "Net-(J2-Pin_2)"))
 (segment (start 173.25 100.5) (end 176.25 97.5) (width 0.2) (layer "F.Cu") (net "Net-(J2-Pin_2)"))
 (segment (start 179.79 72.46) (end 183.185 72.46) (width 0.2) (layer "F.Cu") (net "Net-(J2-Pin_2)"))
 (segment (start 113 97.5) (end 113 99) (width 0.2) (layer "F.Cu") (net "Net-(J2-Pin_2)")))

